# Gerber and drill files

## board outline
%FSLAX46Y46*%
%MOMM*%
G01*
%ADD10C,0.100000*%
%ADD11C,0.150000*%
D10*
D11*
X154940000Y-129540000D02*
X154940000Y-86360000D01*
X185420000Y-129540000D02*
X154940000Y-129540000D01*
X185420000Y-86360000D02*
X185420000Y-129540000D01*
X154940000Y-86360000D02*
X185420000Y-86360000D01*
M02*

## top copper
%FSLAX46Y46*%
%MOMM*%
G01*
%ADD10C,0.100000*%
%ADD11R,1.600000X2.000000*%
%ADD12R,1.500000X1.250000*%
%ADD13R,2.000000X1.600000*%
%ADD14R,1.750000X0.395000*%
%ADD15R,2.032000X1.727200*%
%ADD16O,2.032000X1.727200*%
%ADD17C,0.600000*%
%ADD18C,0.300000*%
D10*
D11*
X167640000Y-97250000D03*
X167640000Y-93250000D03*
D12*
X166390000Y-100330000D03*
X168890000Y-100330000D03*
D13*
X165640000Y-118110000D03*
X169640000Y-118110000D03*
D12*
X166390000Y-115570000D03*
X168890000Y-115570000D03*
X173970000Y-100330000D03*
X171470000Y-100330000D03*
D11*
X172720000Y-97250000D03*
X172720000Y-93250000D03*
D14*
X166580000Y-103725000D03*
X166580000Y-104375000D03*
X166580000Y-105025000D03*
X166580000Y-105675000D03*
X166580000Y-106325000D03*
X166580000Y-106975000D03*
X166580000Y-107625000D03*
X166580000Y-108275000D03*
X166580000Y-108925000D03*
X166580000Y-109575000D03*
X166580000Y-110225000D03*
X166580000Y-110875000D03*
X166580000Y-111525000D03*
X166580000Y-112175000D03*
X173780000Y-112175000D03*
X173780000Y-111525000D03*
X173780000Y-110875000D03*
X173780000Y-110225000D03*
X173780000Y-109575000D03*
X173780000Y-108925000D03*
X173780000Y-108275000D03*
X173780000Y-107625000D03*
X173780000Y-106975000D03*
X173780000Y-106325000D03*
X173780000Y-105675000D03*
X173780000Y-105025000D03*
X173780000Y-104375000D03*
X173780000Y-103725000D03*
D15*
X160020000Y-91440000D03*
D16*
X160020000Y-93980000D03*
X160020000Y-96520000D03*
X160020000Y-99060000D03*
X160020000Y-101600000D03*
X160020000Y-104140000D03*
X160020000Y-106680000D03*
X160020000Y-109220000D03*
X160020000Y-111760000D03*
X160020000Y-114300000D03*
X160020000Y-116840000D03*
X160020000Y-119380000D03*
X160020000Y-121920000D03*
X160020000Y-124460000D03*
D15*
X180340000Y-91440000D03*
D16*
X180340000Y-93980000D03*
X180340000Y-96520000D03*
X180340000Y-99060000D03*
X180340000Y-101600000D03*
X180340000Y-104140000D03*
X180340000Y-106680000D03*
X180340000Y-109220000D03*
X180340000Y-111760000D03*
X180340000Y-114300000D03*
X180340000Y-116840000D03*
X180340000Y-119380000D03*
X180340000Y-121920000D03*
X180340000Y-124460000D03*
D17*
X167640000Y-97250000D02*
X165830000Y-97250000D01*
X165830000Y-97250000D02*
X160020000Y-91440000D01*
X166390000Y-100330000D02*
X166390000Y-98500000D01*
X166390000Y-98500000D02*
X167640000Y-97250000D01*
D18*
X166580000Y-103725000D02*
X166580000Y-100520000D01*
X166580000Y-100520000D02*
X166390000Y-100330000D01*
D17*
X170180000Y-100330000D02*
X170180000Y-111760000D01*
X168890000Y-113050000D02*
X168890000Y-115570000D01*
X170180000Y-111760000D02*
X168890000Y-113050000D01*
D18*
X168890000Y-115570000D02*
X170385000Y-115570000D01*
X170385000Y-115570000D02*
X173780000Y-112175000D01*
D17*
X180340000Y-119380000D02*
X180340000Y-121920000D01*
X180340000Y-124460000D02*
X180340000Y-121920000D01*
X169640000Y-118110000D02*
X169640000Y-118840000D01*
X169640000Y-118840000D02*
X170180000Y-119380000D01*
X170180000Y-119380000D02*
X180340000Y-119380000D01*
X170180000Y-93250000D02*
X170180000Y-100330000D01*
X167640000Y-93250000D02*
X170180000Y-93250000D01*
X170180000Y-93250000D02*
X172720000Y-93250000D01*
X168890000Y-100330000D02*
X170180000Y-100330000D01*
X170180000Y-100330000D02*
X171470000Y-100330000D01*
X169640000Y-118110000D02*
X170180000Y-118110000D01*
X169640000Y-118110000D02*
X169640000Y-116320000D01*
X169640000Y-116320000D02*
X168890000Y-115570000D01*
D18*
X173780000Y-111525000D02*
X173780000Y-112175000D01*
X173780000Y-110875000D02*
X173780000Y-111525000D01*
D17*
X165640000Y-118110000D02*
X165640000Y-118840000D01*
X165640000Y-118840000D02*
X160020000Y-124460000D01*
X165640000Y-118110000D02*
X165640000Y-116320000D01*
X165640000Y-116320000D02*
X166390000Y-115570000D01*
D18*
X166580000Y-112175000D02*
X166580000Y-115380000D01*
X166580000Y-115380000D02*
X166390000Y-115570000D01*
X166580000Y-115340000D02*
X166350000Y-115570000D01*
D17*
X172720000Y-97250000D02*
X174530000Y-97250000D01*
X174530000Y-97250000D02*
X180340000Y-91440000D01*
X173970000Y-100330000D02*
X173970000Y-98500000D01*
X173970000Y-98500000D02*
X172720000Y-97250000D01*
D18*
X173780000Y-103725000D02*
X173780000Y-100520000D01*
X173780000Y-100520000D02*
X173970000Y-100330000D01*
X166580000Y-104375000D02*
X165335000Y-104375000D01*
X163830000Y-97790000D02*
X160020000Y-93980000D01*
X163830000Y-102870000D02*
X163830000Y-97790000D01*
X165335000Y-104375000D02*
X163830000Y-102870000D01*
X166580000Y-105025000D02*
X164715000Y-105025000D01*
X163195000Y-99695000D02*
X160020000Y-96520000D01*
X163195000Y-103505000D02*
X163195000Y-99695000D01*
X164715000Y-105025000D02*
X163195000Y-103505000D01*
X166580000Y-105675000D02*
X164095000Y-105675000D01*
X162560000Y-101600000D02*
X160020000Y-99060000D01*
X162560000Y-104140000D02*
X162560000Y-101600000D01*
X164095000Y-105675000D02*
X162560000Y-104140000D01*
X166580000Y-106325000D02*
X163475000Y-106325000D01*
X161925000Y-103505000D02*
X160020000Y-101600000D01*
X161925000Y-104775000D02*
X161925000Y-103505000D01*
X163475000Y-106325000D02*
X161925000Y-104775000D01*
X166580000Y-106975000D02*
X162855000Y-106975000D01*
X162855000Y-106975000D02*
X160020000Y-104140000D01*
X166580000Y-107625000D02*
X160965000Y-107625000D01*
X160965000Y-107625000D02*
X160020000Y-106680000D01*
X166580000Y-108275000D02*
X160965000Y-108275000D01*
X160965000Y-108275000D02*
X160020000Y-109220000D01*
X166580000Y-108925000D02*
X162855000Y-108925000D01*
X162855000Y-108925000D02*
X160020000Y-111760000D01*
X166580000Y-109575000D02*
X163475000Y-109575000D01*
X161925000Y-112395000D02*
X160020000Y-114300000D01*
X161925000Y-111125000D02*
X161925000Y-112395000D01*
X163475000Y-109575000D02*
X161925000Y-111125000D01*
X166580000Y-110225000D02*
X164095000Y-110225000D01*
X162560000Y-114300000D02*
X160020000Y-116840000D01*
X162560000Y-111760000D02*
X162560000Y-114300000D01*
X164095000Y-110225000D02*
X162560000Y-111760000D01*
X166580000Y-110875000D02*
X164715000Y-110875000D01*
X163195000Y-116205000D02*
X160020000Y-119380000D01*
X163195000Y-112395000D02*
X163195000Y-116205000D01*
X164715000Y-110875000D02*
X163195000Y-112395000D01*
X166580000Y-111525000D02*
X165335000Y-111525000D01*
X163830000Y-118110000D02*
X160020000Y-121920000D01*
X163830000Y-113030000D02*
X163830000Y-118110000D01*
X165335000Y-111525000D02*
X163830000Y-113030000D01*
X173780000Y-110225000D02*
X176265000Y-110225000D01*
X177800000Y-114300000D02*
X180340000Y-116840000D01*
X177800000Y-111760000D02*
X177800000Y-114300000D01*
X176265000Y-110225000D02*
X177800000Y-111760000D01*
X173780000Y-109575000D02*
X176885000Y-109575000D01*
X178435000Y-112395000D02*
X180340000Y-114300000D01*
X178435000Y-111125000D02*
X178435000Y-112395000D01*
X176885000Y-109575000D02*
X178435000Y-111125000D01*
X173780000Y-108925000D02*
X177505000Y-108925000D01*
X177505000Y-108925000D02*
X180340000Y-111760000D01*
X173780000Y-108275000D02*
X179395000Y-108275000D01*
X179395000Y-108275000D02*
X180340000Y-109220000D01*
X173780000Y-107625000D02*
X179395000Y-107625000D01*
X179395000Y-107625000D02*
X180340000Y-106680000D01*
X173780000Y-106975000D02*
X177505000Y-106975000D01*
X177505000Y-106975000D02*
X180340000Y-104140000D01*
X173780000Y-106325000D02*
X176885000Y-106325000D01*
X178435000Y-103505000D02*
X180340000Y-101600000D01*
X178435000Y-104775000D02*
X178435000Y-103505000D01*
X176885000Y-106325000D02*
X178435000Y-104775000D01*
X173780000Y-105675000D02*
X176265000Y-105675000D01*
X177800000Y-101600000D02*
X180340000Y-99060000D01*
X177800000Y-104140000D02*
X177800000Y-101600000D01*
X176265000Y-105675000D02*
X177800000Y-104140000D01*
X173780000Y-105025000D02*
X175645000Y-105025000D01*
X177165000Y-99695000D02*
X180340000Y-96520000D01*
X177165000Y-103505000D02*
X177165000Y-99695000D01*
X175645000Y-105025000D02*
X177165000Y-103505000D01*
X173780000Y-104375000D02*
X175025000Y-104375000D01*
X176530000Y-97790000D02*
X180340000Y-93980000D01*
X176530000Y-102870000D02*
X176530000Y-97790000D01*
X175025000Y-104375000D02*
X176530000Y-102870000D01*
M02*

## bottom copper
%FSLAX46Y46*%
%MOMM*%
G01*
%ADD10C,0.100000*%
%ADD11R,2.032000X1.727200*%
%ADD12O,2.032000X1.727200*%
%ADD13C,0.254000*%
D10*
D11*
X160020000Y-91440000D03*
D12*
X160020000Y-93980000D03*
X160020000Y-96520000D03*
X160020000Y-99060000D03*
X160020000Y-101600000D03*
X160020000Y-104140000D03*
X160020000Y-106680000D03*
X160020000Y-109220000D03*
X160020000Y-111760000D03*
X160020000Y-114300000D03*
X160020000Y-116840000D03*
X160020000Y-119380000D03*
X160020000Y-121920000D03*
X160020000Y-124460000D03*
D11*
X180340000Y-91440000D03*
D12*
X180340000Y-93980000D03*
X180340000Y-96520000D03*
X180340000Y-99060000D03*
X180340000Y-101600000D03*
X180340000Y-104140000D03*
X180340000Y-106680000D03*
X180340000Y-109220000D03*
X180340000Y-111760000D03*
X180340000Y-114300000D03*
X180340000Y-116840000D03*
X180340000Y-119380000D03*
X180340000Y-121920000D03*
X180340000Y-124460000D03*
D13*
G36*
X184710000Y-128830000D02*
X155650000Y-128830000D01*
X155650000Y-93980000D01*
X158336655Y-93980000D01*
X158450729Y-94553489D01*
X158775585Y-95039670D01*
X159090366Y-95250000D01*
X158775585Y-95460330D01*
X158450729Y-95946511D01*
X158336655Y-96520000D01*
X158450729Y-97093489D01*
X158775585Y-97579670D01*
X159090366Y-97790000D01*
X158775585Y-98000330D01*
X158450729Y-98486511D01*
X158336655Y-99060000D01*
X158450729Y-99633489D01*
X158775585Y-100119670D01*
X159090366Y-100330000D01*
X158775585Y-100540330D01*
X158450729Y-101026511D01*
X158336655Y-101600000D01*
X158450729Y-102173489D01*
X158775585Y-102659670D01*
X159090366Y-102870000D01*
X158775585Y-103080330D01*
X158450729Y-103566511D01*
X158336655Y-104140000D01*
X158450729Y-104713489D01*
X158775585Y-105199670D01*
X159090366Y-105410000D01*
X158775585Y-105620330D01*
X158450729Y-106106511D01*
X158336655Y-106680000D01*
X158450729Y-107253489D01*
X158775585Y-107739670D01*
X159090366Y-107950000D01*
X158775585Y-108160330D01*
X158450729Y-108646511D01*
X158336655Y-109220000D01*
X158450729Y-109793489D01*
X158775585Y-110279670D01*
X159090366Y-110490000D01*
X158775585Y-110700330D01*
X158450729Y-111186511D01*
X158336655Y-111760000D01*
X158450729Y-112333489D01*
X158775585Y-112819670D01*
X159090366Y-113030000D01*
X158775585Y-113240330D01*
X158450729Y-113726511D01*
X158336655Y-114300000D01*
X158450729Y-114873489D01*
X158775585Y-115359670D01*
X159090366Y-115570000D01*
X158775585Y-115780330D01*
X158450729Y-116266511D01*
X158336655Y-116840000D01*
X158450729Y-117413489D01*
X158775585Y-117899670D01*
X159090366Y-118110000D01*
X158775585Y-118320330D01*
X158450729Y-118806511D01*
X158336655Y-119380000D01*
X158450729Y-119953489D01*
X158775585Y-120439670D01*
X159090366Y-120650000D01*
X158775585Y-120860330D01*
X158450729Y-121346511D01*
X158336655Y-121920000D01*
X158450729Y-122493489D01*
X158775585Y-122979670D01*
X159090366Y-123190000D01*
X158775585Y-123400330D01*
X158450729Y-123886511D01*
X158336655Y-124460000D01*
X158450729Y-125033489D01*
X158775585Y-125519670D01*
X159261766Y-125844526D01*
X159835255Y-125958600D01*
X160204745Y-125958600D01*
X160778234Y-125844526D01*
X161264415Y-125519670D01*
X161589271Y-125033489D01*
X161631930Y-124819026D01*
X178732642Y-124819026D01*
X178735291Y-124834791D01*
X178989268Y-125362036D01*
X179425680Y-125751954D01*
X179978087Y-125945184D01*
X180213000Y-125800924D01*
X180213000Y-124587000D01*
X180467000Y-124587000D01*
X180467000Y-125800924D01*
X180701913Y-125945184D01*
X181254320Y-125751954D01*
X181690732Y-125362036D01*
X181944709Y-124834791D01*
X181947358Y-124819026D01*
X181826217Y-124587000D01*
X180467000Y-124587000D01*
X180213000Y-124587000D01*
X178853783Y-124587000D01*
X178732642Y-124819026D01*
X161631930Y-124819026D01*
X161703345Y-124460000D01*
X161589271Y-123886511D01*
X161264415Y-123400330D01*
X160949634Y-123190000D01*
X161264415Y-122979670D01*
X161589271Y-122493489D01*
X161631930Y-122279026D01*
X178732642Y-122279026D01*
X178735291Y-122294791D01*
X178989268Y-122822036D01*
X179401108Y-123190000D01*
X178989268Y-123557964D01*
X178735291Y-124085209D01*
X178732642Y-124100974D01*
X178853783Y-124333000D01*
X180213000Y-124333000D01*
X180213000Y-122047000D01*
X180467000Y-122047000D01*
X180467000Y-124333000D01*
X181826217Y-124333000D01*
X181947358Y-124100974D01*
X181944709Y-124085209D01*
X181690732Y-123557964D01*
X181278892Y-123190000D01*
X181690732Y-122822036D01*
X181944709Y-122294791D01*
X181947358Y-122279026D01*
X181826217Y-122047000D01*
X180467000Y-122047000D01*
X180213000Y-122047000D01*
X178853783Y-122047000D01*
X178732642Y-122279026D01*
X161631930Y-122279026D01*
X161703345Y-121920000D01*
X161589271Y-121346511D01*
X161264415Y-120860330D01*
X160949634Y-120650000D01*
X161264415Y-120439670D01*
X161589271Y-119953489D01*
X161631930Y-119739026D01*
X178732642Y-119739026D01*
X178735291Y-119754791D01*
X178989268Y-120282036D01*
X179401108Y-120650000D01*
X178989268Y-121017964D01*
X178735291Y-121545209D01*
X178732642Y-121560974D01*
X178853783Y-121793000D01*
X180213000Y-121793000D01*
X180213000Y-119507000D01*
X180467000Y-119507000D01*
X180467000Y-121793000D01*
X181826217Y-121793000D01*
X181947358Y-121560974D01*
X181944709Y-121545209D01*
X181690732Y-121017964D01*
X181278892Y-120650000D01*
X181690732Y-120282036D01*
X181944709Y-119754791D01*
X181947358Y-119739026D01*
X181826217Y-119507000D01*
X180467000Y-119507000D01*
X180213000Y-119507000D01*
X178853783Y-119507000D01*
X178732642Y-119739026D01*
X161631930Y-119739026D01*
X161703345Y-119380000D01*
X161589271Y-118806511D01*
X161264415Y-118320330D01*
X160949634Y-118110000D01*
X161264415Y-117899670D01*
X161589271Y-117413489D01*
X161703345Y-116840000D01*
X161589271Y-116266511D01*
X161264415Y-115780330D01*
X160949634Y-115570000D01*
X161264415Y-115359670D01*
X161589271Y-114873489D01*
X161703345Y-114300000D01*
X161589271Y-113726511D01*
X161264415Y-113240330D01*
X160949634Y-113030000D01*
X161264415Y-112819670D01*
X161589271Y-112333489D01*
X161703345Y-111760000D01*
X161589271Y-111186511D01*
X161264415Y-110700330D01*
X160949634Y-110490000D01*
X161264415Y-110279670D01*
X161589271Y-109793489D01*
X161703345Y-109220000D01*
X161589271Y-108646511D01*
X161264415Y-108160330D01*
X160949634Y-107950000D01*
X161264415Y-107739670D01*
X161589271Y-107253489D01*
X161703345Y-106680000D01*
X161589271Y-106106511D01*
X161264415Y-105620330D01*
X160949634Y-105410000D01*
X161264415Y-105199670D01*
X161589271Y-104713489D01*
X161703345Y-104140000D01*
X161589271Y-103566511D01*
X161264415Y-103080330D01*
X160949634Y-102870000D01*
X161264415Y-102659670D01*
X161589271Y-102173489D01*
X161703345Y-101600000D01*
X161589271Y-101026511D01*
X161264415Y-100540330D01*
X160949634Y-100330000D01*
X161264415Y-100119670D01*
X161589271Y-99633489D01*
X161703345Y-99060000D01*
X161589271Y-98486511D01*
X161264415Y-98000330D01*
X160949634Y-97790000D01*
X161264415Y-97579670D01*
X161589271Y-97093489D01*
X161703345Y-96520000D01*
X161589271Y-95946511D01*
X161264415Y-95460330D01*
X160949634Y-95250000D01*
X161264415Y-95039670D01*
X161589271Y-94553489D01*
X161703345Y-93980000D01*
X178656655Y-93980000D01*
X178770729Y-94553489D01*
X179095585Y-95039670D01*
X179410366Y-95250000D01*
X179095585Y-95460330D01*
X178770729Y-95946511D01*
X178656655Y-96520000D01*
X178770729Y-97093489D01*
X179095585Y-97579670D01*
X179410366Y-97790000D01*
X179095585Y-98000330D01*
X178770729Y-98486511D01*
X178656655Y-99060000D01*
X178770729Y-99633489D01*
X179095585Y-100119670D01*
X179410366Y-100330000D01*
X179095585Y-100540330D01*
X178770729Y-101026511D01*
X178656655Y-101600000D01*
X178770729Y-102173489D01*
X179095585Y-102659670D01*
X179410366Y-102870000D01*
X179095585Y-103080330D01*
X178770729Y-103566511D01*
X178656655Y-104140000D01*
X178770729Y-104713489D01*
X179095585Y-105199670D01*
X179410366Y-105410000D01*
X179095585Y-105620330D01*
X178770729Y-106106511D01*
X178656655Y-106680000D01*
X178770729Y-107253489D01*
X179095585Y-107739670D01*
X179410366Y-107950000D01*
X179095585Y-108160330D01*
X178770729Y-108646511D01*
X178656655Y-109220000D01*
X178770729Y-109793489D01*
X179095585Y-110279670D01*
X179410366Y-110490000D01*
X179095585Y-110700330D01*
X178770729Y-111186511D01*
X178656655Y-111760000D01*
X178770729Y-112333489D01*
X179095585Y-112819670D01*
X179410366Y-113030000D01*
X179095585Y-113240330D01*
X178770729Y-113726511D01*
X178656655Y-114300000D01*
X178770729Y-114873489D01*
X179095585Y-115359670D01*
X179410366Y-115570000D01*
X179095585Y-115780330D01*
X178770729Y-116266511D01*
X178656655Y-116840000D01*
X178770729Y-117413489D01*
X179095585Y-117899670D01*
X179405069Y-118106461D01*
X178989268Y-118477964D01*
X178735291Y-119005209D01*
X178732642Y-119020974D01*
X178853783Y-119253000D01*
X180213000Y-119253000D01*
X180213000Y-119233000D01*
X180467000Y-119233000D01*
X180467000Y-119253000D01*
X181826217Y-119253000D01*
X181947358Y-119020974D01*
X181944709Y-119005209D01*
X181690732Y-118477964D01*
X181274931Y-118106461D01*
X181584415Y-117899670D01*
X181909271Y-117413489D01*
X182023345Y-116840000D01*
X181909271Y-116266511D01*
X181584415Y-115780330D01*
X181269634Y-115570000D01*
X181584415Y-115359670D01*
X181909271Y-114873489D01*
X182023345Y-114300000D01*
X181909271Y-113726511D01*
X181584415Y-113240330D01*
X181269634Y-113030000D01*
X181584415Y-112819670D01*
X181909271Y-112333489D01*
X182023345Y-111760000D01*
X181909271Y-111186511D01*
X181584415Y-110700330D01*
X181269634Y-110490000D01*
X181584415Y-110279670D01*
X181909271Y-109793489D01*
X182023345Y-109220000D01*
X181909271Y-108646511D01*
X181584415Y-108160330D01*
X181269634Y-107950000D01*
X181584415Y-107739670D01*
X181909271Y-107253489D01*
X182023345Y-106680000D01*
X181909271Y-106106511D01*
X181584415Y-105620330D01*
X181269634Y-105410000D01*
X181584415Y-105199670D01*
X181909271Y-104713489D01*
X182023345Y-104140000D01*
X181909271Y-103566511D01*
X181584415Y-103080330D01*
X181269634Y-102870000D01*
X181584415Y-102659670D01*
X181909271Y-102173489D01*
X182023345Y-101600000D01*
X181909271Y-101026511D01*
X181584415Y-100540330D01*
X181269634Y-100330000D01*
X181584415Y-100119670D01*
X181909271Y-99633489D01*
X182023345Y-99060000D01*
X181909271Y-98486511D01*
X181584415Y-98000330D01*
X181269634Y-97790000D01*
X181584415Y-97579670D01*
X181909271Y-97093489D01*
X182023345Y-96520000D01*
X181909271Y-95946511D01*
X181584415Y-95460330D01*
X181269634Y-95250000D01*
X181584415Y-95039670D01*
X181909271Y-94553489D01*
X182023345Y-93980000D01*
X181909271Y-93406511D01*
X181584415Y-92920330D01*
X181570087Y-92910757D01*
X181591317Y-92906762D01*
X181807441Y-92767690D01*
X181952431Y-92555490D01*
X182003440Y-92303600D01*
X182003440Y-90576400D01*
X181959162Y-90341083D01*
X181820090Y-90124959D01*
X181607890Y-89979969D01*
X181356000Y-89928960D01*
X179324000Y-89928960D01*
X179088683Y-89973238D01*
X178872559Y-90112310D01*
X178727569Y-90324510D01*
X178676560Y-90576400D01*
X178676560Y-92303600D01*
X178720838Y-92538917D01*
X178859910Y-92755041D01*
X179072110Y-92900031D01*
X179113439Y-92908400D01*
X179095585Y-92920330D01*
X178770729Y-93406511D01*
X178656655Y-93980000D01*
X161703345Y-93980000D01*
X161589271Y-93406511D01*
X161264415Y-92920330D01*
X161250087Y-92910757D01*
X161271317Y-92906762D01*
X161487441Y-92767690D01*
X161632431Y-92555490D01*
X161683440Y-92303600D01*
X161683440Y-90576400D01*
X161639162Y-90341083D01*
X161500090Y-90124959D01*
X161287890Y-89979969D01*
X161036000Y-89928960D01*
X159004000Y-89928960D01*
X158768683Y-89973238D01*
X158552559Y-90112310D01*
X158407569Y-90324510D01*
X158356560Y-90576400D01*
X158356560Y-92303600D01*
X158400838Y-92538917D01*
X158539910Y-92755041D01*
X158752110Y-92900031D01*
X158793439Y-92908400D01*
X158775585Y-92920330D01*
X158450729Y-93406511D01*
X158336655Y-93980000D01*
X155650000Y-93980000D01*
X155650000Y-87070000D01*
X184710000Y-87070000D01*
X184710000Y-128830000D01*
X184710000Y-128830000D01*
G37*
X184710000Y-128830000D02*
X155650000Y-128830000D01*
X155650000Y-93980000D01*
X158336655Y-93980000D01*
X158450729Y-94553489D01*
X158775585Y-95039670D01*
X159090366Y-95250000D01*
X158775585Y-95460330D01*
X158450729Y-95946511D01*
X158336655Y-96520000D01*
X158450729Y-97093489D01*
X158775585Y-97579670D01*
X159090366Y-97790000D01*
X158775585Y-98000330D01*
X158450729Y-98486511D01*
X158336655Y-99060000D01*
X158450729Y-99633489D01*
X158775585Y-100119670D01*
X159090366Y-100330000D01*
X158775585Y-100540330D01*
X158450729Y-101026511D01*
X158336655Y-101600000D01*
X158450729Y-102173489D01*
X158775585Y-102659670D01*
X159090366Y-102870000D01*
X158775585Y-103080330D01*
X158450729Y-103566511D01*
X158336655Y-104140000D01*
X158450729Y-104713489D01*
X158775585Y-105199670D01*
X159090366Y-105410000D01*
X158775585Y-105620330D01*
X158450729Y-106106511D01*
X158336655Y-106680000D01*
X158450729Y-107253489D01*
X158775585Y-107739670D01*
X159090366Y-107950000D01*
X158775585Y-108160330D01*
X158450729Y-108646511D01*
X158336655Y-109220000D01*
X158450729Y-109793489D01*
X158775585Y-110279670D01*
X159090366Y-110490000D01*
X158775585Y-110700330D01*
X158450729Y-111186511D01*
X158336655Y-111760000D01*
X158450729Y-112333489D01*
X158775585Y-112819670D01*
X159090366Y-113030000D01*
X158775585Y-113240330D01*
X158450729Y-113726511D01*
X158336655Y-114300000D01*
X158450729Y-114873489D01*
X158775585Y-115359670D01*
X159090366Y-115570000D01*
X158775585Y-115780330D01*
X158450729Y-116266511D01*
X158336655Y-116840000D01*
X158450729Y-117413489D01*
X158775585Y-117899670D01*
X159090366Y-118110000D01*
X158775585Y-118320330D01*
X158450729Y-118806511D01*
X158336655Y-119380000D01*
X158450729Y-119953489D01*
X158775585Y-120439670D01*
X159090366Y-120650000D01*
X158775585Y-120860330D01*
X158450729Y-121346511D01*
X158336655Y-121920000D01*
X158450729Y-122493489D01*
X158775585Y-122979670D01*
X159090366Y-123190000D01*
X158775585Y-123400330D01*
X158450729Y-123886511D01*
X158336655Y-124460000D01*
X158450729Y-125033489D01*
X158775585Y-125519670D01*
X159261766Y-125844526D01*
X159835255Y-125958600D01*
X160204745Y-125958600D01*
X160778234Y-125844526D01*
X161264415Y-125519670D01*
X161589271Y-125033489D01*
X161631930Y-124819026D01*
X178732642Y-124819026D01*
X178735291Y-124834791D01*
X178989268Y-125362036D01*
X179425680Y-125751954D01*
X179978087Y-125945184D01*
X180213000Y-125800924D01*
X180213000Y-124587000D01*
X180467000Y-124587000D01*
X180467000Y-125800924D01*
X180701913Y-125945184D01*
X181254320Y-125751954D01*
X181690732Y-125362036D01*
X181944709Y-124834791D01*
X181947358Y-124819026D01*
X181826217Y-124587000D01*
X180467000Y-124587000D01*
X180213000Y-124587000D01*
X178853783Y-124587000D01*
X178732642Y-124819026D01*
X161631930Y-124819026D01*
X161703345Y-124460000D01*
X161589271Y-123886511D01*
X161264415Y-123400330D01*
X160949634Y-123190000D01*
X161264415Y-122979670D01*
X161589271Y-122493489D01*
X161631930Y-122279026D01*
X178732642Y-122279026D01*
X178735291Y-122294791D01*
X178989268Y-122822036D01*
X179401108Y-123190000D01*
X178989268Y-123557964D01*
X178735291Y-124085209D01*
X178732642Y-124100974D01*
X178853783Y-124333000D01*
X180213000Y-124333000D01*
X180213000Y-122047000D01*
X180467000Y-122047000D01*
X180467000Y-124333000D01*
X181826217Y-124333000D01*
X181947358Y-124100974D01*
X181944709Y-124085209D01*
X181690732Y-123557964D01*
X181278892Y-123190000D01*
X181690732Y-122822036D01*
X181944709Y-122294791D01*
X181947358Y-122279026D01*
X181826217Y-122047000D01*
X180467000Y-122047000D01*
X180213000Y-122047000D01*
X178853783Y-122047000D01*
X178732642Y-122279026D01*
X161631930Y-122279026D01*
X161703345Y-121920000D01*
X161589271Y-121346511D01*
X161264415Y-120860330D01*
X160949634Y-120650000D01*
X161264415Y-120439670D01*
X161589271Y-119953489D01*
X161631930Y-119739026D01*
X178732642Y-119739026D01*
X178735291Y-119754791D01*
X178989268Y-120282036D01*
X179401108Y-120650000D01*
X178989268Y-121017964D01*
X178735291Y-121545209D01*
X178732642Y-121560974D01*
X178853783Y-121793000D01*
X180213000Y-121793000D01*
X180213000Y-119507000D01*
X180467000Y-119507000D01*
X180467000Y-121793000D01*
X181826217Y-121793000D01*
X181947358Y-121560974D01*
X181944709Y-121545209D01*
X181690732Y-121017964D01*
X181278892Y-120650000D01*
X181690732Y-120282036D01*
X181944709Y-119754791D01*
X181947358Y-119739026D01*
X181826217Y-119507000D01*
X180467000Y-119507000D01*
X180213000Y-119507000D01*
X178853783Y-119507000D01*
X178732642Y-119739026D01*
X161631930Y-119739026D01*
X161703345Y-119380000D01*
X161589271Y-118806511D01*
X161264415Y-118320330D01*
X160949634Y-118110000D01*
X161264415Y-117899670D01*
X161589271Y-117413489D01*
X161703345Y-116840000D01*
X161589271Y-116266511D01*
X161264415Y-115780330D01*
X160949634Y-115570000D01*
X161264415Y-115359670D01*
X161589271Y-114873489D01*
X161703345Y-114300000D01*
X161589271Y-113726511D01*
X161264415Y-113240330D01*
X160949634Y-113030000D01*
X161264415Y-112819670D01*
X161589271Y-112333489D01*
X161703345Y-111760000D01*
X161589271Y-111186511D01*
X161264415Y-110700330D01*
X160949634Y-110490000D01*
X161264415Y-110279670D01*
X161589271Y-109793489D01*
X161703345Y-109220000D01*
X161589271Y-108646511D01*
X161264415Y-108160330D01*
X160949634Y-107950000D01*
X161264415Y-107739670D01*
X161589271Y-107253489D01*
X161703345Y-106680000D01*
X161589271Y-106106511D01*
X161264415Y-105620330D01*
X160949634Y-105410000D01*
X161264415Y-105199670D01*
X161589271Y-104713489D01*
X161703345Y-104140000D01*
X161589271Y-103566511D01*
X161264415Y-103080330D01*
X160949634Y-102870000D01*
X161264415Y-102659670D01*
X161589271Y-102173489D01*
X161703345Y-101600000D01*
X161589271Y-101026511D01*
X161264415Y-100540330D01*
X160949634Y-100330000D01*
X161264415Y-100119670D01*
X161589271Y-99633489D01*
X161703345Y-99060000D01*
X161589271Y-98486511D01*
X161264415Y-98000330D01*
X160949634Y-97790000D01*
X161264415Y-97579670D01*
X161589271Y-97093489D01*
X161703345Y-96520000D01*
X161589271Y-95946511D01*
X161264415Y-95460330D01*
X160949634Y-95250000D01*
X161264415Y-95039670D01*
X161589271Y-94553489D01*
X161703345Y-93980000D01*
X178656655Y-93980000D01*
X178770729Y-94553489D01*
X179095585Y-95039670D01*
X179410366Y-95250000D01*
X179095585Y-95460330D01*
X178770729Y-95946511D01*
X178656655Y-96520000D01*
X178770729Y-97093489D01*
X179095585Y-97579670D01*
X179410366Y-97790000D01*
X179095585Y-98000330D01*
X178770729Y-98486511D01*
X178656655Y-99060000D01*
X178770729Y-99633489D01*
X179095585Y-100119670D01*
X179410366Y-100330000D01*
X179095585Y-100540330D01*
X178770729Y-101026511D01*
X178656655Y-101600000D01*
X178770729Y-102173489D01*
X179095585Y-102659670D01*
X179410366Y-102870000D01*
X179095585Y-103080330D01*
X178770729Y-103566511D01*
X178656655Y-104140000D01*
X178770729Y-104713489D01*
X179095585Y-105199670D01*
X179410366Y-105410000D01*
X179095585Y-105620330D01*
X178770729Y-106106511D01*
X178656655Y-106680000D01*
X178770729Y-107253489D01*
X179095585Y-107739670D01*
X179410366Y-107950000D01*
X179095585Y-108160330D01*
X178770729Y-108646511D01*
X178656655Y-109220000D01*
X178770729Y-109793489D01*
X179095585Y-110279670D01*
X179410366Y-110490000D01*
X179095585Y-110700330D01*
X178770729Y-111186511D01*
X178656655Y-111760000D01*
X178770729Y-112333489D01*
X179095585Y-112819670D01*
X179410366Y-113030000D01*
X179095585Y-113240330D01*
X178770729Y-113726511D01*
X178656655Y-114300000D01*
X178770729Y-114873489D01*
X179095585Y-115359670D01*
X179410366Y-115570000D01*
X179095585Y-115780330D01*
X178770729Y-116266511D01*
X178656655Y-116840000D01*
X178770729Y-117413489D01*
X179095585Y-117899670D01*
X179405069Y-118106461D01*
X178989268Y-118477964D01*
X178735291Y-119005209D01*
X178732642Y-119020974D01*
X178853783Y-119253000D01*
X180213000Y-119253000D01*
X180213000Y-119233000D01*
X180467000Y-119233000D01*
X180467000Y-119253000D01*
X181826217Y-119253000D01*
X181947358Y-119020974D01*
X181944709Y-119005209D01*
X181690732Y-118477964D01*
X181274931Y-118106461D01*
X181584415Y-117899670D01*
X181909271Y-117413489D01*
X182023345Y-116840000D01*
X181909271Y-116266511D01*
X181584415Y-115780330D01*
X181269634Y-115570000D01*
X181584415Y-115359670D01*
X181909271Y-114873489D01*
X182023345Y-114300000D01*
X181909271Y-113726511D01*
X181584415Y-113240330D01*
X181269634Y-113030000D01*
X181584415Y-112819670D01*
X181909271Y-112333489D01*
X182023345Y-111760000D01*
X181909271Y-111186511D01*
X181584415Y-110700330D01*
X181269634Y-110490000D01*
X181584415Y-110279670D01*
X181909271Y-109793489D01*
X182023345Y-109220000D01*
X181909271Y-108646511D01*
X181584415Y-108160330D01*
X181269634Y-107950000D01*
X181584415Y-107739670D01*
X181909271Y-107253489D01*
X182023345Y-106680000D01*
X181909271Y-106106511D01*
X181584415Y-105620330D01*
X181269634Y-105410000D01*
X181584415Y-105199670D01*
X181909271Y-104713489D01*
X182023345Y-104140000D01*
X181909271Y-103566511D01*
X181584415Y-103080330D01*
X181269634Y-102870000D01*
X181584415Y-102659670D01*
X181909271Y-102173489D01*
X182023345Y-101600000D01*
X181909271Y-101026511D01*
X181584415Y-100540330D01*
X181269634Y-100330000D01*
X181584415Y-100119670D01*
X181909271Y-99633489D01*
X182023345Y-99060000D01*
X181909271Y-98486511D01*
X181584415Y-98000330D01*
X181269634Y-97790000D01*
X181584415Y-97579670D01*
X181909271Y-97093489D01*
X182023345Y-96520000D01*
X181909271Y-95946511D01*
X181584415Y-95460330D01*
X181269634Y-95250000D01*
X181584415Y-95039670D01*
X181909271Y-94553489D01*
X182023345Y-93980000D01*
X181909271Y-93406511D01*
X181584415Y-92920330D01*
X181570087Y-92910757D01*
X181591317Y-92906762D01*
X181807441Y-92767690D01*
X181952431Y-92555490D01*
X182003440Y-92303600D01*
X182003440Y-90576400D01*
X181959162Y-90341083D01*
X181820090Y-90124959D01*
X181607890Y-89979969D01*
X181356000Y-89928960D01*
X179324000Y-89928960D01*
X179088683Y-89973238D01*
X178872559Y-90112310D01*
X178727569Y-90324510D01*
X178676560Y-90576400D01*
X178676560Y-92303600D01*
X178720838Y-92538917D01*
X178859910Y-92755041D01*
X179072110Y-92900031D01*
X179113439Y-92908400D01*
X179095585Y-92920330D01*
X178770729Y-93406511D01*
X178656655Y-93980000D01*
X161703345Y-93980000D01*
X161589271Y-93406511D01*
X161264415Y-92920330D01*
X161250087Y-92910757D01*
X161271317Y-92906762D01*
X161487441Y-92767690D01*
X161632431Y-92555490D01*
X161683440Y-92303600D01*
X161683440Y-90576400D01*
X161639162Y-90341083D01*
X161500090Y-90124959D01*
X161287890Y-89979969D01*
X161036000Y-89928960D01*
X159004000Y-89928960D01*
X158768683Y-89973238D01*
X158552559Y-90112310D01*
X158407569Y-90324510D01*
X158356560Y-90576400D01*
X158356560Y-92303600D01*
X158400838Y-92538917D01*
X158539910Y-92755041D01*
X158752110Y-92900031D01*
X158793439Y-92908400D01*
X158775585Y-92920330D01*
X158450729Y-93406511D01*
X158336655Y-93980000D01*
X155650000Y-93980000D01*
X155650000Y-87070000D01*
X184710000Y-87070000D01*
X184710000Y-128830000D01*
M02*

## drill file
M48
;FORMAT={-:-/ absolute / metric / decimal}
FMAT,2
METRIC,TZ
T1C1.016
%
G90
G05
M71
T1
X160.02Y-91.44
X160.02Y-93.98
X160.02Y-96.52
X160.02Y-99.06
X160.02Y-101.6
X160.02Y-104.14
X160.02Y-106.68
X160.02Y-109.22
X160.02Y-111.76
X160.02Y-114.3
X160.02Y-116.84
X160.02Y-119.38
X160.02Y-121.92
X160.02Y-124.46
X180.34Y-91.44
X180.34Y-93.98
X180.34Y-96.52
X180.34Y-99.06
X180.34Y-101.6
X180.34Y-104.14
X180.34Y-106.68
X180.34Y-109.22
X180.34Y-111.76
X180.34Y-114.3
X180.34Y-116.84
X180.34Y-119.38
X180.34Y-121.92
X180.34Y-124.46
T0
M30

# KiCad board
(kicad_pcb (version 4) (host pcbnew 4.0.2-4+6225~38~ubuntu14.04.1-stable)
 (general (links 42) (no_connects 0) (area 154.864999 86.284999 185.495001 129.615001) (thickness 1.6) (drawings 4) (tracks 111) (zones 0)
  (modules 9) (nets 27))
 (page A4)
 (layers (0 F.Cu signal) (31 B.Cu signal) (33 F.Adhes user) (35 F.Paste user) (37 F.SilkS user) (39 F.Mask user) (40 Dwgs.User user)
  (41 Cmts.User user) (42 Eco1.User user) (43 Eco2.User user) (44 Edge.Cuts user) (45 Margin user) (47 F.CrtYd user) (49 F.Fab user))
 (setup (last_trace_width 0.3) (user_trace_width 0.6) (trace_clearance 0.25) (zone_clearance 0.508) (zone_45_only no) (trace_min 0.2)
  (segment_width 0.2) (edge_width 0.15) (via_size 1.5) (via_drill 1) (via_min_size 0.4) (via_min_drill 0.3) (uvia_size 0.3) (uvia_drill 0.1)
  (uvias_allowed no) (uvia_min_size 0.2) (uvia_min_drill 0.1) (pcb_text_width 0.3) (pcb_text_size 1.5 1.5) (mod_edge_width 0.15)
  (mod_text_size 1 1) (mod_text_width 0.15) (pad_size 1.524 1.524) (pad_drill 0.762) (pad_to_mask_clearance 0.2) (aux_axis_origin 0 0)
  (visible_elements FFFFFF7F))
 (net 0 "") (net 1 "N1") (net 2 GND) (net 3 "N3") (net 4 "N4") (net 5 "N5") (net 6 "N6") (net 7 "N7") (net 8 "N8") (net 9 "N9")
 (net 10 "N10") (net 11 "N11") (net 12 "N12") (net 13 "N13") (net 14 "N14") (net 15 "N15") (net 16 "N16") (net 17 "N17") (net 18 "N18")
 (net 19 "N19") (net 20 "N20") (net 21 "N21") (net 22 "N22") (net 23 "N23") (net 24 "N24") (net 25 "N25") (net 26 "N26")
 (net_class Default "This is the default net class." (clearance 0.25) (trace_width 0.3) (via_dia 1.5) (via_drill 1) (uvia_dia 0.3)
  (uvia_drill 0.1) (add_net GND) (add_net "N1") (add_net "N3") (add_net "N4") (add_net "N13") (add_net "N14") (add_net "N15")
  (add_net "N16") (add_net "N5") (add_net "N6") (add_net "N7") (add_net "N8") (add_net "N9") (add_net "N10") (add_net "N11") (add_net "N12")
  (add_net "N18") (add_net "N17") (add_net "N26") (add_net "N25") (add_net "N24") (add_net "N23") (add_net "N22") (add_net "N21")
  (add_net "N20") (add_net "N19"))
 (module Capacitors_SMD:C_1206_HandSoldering (layer F.Cu) (at 167.64 95.25 90)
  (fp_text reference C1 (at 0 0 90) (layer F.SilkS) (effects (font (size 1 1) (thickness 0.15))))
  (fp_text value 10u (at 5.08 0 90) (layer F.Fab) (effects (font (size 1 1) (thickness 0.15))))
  (pad 1 smd rect (at -2 0 90) (size 2 1.6) (layers F.Cu F.Paste F.Mask) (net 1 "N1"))
  (pad 2 smd rect (at 2 0 90) (size 2 1.6) (layers F.Cu F.Paste F.Mask) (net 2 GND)))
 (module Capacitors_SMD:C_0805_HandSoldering (layer F.Cu) (at 167.64 100.33)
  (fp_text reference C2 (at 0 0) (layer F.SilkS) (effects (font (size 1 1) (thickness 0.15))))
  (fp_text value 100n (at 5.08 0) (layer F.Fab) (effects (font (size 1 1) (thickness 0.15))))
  (pad 1 smd rect (at -1.25 0) (size 1.5 1.25) (layers F.Cu F.Paste F.Mask) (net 1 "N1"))
  (pad 2 smd rect (at 1.25 0) (size 1.5 1.25) (layers F.Cu F.Paste F.Mask) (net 2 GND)))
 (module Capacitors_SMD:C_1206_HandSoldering (layer F.Cu) (at 167.64 118.11)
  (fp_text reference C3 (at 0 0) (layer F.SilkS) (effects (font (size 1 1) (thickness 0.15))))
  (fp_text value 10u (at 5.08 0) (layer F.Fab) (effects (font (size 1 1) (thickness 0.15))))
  (pad 1 smd rect (at -2 0) (size 2 1.6) (layers F.Cu F.Paste F.Mask) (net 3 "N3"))
  (pad 2 smd rect (at 2 0) (size 2 1.6) (layers F.Cu F.Paste F.Mask) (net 2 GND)))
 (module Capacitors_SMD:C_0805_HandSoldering (layer F.Cu) (at 167.64 115.57)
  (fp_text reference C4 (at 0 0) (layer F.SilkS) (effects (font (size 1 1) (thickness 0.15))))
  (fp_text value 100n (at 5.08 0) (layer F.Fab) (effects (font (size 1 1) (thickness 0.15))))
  (pad 1 smd rect (at -1.25 0) (size 1.5 1.25) (layers F.Cu F.Paste F.Mask) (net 3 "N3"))
  (pad 2 smd rect (at 1.25 0) (size 1.5 1.25) (layers F.Cu F.Paste F.Mask) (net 2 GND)))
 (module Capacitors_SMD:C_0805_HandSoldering (layer F.Cu) (at 172.72 100.33 180)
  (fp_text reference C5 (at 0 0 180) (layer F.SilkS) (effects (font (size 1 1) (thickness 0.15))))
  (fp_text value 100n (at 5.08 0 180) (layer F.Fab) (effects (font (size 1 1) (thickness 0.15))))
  (pad 1 smd rect (at -1.25 0 180) (size 1.5 1.25) (layers F.Cu F.Paste F.Mask) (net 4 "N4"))
  (pad 2 smd rect (at 1.25 0 180) (size 1.5 1.25) (layers F.Cu F.Paste F.Mask) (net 2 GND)))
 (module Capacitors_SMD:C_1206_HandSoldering (layer F.Cu) (at 172.72 95.25 90)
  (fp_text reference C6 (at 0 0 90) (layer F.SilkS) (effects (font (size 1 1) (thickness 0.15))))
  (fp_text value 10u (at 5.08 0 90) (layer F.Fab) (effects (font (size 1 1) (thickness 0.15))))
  (pad 1 smd rect (at -2 0 90) (size 2 1.6) (layers F.Cu F.Paste F.Mask) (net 4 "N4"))
  (pad 2 smd rect (at 2 0 90) (size 2 1.6) (layers F.Cu F.Paste F.Mask) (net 2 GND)))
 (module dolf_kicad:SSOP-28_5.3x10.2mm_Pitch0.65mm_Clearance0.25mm (layer F.Cu) (at 170.18 107.95)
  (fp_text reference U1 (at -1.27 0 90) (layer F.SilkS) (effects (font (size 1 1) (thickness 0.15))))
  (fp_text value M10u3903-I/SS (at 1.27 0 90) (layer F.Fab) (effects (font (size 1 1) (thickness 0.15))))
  (pad 1 smd rect (at -3.6 -4.225) (size 1.75 0.395) (layers F.Cu F.Paste F.Mask) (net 1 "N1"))
  (pad 2 smd rect (at -3.6 -3.575) (size 1.75 0.395) (layers F.Cu F.Paste F.Mask) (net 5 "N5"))
  (pad 3 smd rect (at -3.6 -2.925) (size 1.75 0.395) (layers F.Cu F.Paste F.Mask) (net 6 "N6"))
  (pad 4 smd rect (at -3.6 -2.275) (size 1.75 0.395) (layers F.Cu F.Paste F.Mask) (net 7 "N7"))
  (pad 5 smd rect (at -3.6 -1.625) (size 1.75 0.395) (layers F.Cu F.Paste F.Mask) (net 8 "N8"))
  (pad 6 smd rect (at -3.6 -0.975) (size 1.75 0.395) (layers F.Cu F.Paste F.Mask) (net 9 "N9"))
  (pad 7 smd rect (at -3.6 -0.325) (size 1.75 0.395) (layers F.Cu F.Paste F.Mask) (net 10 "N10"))
  (pad 8 smd rect (at -3.6 0.325) (size 1.75 0.395) (layers F.Cu F.Paste F.Mask) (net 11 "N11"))
  (pad 9 smd rect (at -3.6 0.975) (size 1.75 0.395) (layers F.Cu F.Paste F.Mask) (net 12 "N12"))
  (pad 10 smd rect (at -3.6 1.625) (size 1.75 0.395) (layers F.Cu F.Paste F.Mask) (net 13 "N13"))
  (pad 11 smd rect (at -3.6 2.275) (size 1.75 0.395) (layers F.Cu F.Paste F.Mask) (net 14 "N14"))
  (pad 12 smd rect (at -3.6 2.925) (size 1.75 0.395) (layers F.Cu F.Paste F.Mask) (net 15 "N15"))
  (pad 13 smd rect (at -3.6 3.575) (size 1.75 0.395) (layers F.Cu F.Paste F.Mask) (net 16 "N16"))
  (pad 14 smd rect (at -3.6 4.225) (size 1.75 0.395) (layers F.Cu F.Paste F.Mask) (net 3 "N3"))
  (pad 15 smd rect (at 3.6 4.225) (size 1.75 0.395) (layers F.Cu F.Paste F.Mask) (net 2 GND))
  (pad 16 smd rect (at 3.6 3.575) (size 1.75 0.395) (layers F.Cu F.Paste F.Mask) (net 2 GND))
  (pad 17 smd rect (at 3.6 2.925) (size 1.75 0.395) (layers F.Cu F.Paste F.Mask) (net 2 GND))
  (pad 18 smd rect (at 3.6 2.275) (size 1.75 0.395) (layers F.Cu F.Paste F.Mask) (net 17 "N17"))
  (pad 19 smd rect (at 3.6 1.625) (size 1.75 0.395) (layers F.Cu F.Paste F.Mask) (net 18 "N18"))
  (pad 20 smd rect (at 3.6 0.975) (size 1.75 0.395) (layers F.Cu F.Paste F.Mask) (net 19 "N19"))
  (pad 21 smd rect (at 3.6 0.325) (size 1.75 0.395) (layers F.Cu F.Paste F.Mask) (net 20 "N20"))
  (pad 22 smd rect (at 3.6 -0.325) (size 1.75 0.395) (layers F.Cu F.Paste F.Mask) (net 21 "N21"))
  (pad 23 smd rect (at 3.6 -0.975) (size 1.75 0.395) (layers F.Cu F.Paste F.Mask) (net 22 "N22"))
  (pad 24 smd rect (at 3.6 -1.625) (size 1.75 0.395) (layers F.Cu F.Paste F.Mask) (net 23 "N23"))
  (pad 25 smd rect (at 3.6 -2.275) (size 1.75 0.395) (layers F.Cu F.Paste F.Mask) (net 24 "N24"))
  (pad 26 smd rect (at 3.6 -2.925) (size 1.75 0.395) (layers F.Cu F.Paste F.Mask) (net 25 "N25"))
  (pad 27 smd rect (at 3.6 -3.575) (size 1.75 0.395) (layers F.Cu F.Paste F.Mask) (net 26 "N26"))
  (pad 28 smd rect (at 3.6 -4.225) (size 1.75 0.395) (layers F.Cu F.Paste F.Mask) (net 4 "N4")))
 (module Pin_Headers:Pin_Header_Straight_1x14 (layer F.Cu) (at 160.02 91.44)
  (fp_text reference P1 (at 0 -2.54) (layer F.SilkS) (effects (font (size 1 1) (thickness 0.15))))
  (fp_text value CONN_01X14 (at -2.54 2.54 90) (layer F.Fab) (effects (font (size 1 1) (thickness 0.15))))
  (pad 1 thru_hole rect (at 0 0) (size 2.032 1.7272) (drill 1.016) (layers *.Cu *.Mask F.SilkS) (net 1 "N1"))
  (pad 2 thru_hole oval (at 0 2.54) (size 2.032 1.7272) (drill 1.016) (layers *.Cu *.Mask F.SilkS) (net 5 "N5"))
  (pad 3 thru_hole oval (at 0 5.08) (size 2.032 1.7272) (drill 1.016) (layers *.Cu *.Mask F.SilkS) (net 6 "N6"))
  (pad 4 thru_hole oval (at 0 7.62) (size 2.032 1.7272) (drill 1.016) (layers *.Cu *.Mask F.SilkS) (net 7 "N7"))
  (pad 5 thru_hole oval (at 0 10.16) (size 2.032 1.7272) (drill 1.016) (layers *.Cu *.Mask F.SilkS) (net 8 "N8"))
  (pad 6 thru_hole oval (at 0 12.7) (size 2.032 1.7272) (drill 1.016) (layers *.Cu *.Mask F.SilkS) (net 9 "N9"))
  (pad 7 thru_hole oval (at 0 15.24) (size 2.032 1.7272) (drill 1.016) (layers *.Cu *.Mask F.SilkS) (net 10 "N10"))
  (pad 8 thru_hole oval (at 0 17.78) (size 2.032 1.7272) (drill 1.016) (layers *.Cu *.Mask F.SilkS) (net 11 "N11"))
  (pad 9 thru_hole oval (at 0 20.32) (size 2.032 1.7272) (drill 1.016) (layers *.Cu *.Mask F.SilkS) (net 12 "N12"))
  (pad 10 thru_hole oval (at 0 22.86) (size 2.032 1.7272) (drill 1.016) (layers *.Cu *.Mask F.SilkS) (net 13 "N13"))
  (pad 11 thru_hole oval (at 0 25.4) (size 2.032 1.7272) (drill 1.016) (layers *.Cu *.Mask F.SilkS) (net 14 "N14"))
  (pad 12 thru_hole oval (at 0 27.94) (size 2.032 1.7272) (drill 1.016) (layers *.Cu *.Mask F.SilkS) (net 15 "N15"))
  (pad 13 thru_hole oval (at 0 30.48) (size 2.032 1.7272) (drill 1.016) (layers *.Cu *.Mask F.SilkS) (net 16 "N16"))
  (pad 14 thru_hole oval (at 0 33.02) (size 2.032 1.7272) (drill 1.016) (layers *.Cu *.Mask F.SilkS) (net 3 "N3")))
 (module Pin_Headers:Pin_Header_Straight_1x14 (layer F.Cu) (at 180.34 91.44)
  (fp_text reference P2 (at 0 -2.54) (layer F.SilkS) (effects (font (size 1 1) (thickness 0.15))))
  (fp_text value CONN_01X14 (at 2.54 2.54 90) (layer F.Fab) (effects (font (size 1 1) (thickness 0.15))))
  (pad 1 thru_hole rect (at 0 0) (size 2.032 1.7272) (drill 1.016) (layers *.Cu *.Mask F.SilkS) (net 4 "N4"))
  (pad 2 thru_hole oval (at 0 2.54) (size 2.032 1.7272) (drill 1.016) (layers *.Cu *.Mask F.SilkS) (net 26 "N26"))
  (pad 3 thru_hole oval (at 0 5.08) (size 2.032 1.7272) (drill 1.016) (layers *.Cu *.Mask F.SilkS) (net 25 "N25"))
  (pad 4 thru_hole oval (at 0 7.62) (size 2.032 1.7272) (drill 1.016) (layers *.Cu *.Mask F.SilkS) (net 24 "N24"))
  (pad 5 thru_hole oval (at 0 10.16) (size 2.032 1.7272) (drill 1.016) (layers *.Cu *.Mask F.SilkS) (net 23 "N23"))
  (pad 6 thru_hole oval (at 0 12.7) (size 2.032 1.7272) (drill 1.016) (layers *.Cu *.Mask F.SilkS) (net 22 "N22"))
  (pad 7 thru_hole oval (at 0 15.24) (size 2.032 1.7272) (drill 1.016) (layers *.Cu *.Mask F.SilkS) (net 21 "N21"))
  (pad 8 thru_hole oval (at 0 17.78) (size 2.032 1.7272) (drill 1.016) (layers *.Cu *.Mask F.SilkS) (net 20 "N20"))
  (pad 9 thru_hole oval (at 0 20.32) (size 2.032 1.7272) (drill 1.016) (layers *.Cu *.Mask F.SilkS) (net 19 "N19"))
  (pad 10 thru_hole oval (at 0 22.86) (size 2.032 1.7272) (drill 1.016) (layers *.Cu *.Mask F.SilkS) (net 18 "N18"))
  (pad 11 thru_hole oval (at 0 25.4) (size 2.032 1.7272) (drill 1.016) (layers *.Cu *.Mask F.SilkS) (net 17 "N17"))
  (pad 12 thru_hole oval (at 0 27.94) (size 2.032 1.7272) (drill 1.016) (layers *.Cu *.Mask F.SilkS) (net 2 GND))
  (pad 13 thru_hole oval (at 0 30.48) (size 2.032 1.7272) (drill 1.016) (layers *.Cu *.Mask F.SilkS) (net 2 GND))
  (pad 14 thru_hole oval (at 0 33.02) (size 2.032 1.7272) (drill 1.016) (layers *.Cu *.Mask F.SilkS) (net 2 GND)))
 (gr_line (start 154.94 129.54) (end 154.94 86.36) (angle 90) (layer Edge.Cuts) (width 0.15))
 (gr_line (start 185.42 129.54) (end 154.94 129.54) (angle 90) (layer Edge.Cuts) (width 0.15))
 (gr_line (start 185.42 86.36) (end 185.42 129.54) (angle 90) (layer Edge.Cuts) (width 0.15))
 (gr_line (start 154.94 86.36) (end 185.42 86.36) (angle 90) (layer Edge.Cuts) (width 0.15))
 (segment (start 167.64 97.25) (end 165.83 97.25) (width 0.6) (layer F.Cu) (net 1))
 (segment (start 165.83 97.25) (end 160.02 91.44) (width 0.6) (layer F.Cu) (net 1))
 (segment (start 166.39 100.33) (end 166.39 98.5) (width 0.6) (layer F.Cu) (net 1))
 (segment (start 166.39 98.5) (end 167.64 97.25) (width 0.6) (layer F.Cu) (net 1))
 (segment (start 166.58 103.725) (end 166.58 100.52) (width 0.3) (layer F.Cu) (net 1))
 (segment (start 166.58 100.52) (end 166.39 100.33) (width 0.3) (layer F.Cu) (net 1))
 (segment (start 170.18 100.33) (end 170.18 111.76) (width 0.6) (layer F.Cu) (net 2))
 (segment (start 168.89 113.05) (end 168.89 115.57) (width 0.6) (layer F.Cu) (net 2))
 (segment (start 170.18 111.76) (end 168.89 113.05) (width 0.6) (layer F.Cu) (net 2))
 (segment (start 168.89 115.57) (end 170.385 115.57) (width 0.3) (layer F.Cu) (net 2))
 (segment (start 170.385 115.57) (end 173.78 112.175) (width 0.3) (layer F.Cu) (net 2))
 (segment (start 180.34 119.38) (end 180.34 121.92) (width 0.6) (layer F.Cu) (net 2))
 (segment (start 180.34 124.46) (end 180.34 121.92) (width 0.6) (layer F.Cu) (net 2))
 (segment (start 169.64 118.11) (end 169.64 118.84) (width 0.6) (layer F.Cu) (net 2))
 (segment (start 169.64 118.84) (end 170.18 119.38) (width 0.6) (layer F.Cu) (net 2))
 (segment (start 170.18 119.38) (end 180.34 119.38) (width 0.6) (layer F.Cu) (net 2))
 (segment (start 170.18 93.25) (end 170.18 100.33) (width 0.6) (layer F.Cu) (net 2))
 (segment (start 167.64 93.25) (end 170.18 93.25) (width 0.6) (layer F.Cu) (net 2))
 (segment (start 170.18 93.25) (end 172.72 93.25) (width 0.6) (layer F.Cu) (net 2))
 (segment (start 168.89 100.33) (end 170.18 100.33) (width 0.6) (layer F.Cu) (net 2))
 (segment (start 170.18 100.33) (end 171.47 100.33) (width 0.6) (layer F.Cu) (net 2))
 (segment (start 169.64 118.11) (end 170.18 118.11) (width 0.6) (layer F.Cu) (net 2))
 (segment (start 169.64 118.11) (end 169.64 116.32) (width 0.6) (layer F.Cu) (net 2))
 (segment (start 169.64 116.32) (end 168.89 115.57) (width 0.6) (layer F.Cu) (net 2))
 (segment (start 173.78 111.525) (end 173.78 112.175) (width 0.3) (layer F.Cu) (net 2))
 (segment (start 173.78 110.875) (end 173.78 111.525) (width 0.3) (layer F.Cu) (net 2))
 (segment (start 165.64 118.11) (end 165.64 118.84) (width 0.6) (layer F.Cu) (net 3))
 (segment (start 165.64 118.84) (end 160.02 124.46) (width 0.6) (layer F.Cu) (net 3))
 (segment (start 165.64 118.11) (end 165.64 116.32) (width 0.6) (layer F.Cu) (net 3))
 (segment (start 165.64 116.32) (end 166.39 115.57) (width 0.6) (layer F.Cu) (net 3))
 (segment (start 166.58 112.175) (end 166.58 115.38) (width 0.3) (layer F.Cu) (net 3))
 (segment (start 166.58 115.38) (end 166.39 115.57) (width 0.3) (layer F.Cu) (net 3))
 (segment (start 166.58 115.34) (end 166.35 115.57) (width 0.3) (layer F.Cu) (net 3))
 (segment (start 172.72 97.25) (end 174.53 97.25) (width 0.6) (layer F.Cu) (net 4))
 (segment (start 174.53 97.25) (end 180.34 91.44) (width 0.6) (layer F.Cu) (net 4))
 (segment (start 173.97 100.33) (end 173.97 98.5) (width 0.6) (layer F.Cu) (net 4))
 (segment (start 173.97 98.5) (end 172.72 97.25) (width 0.6) (layer F.Cu) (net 4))
 (segment (start 173.78 103.725) (end 173.78 100.52) (width 0.3) (layer F.Cu) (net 4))
 (segment (start 173.78 100.52) (end 173.97 100.33) (width 0.3) (layer F.Cu) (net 4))
 (segment (start 166.58 104.375) (end 165.335 104.375) (width 0.3) (layer F.Cu) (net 5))
 (segment (start 163.83 97.79) (end 160.02 93.98) (width 0.3) (layer F.Cu) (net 5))
 (segment (start 163.83 102.87) (end 163.83 97.79) (width 0.3) (layer F.Cu) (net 5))
 (segment (start 165.335 104.375) (end 163.83 102.87) (width 0.3) (layer F.Cu) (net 5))
 (segment (start 166.58 105.025) (end 164.715 105.025) (width 0.3) (layer F.Cu) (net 6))
 (segment (start 163.195 99.695) (end 160.02 96.52) (width 0.3) (layer F.Cu) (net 6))
 (segment (start 163.195 103.505) (end 163.195 99.695) (width 0.3) (layer F.Cu) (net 6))
 (segment (start 164.715 105.025) (end 163.195 103.505) (width 0.3) (layer F.Cu) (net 6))
 (segment (start 166.58 105.675) (end 164.095 105.675) (width 0.3) (layer F.Cu) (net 7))
 (segment (start 162.56 101.6) (end 160.02 99.06) (width 0.3) (layer F.Cu) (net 7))
 (segment (start 162.56 104.14) (end 162.56 101.6) (width 0.3) (layer F.Cu) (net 7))
 (segment (start 164.095 105.675) (end 162.56 104.14) (width 0.3) (layer F.Cu) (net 7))
 (segment (start 166.58 106.325) (end 163.475 106.325) (width 0.3) (layer F.Cu) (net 8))
 (segment (start 161.925 103.505) (end 160.02 101.6) (width 0.3) (layer F.Cu) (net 8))
 (segment (start 161.925 104.775) (end 161.925 103.505) (width 0.3) (layer F.Cu) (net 8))
 (segment (start 163.475 106.325) (end 161.925 104.775) (width 0.3) (layer F.Cu) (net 8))
 (segment (start 166.58 106.975) (end 162.855 106.975) (width 0.3) (layer F.Cu) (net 9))
 (segment (start 162.855 106.975) (end 160.02 104.14) (width 0.3) (layer F.Cu) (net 9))
 (segment (start 166.58 107.625) (end 160.965 107.625) (width 0.3) (layer F.Cu) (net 10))
 (segment (start 160.965 107.625) (end 160.02 106.68) (width 0.3) (layer F.Cu) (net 10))
 (segment (start 166.58 108.275) (end 160.965 108.275) (width 0.3) (layer F.Cu) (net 11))
 (segment (start 160.965 108.275) (end 160.02 109.22) (width 0.3) (layer F.Cu) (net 11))
 (segment (start 166.58 108.925) (end 162.855 108.925) (width 0.3) (layer F.Cu) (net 12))
 (segment (start 162.855 108.925) (end 160.02 111.76) (width 0.3) (layer F.Cu) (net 12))
 (segment (start 166.58 109.575) (end 163.475 109.575) (width 0.3) (layer F.Cu) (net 13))
 (segment (start 161.925 112.395) (end 160.02 114.3) (width 0.3) (layer F.Cu) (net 13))
 (segment (start 161.925 111.125) (end 161.925 112.395) (width 0.3) (layer F.Cu) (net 13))
 (segment (start 163.475 109.575) (end 161.925 111.125) (width 0.3) (layer F.Cu) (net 13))
 (segment (start 166.58 110.225) (end 164.095 110.225) (width 0.3) (layer F.Cu) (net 14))
 (segment (start 162.56 114.3) (end 160.02 116.84) (width 0.3) (layer F.Cu) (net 14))
 (segment (start 162.56 111.76) (end 162.56 114.3) (width 0.3) (layer F.Cu) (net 14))
 (segment (start 164.095 110.225) (end 162.56 111.76) (width 0.3) (layer F.Cu) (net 14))
 (segment (start 166.58 110.875) (end 164.715 110.875) (width 0.3) (layer F.Cu) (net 15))
 (segment (start 163.195 116.205) (end 160.02 119.38) (width 0.3) (layer F.Cu) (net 15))
 (segment (start 163.195 112.395) (end 163.195 116.205) (width 0.3) (layer F.Cu) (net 15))
 (segment (start 164.715 110.875) (end 163.195 112.395) (width 0.3) (layer F.Cu) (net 15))
 (segment (start 166.58 111.525) (end 165.335 111.525) (width 0.3) (layer F.Cu) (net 16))
 (segment (start 163.83 118.11) (end 160.02 121.92) (width 0.3) (layer F.Cu) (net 16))
 (segment (start 163.83 113.03) (end 163.83 118.11) (width 0.3) (layer F.Cu) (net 16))
 (segment (start 165.335 111.525) (end 163.83 113.03) (width 0.3) (layer F.Cu) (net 16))
 (segment (start 173.78 110.225) (end 176.265 110.225) (width 0.3) (layer F.Cu) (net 17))
 (segment (start 177.8 114.3) (end 180.34 116.84) (width 0.3) (layer F.Cu) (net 17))
 (segment (start 177.8 111.76) (end 177.8 114.3) (width 0.3) (layer F.Cu) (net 17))
 (segment (start 176.265 110.225) (end 177.8 111.76) (width 0.3) (layer F.Cu) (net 17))
 (segment (start 173.78 109.575) (end 176.885 109.575) (width 0.3) (layer F.Cu) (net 18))
 (segment (start 178.435 112.395) (end 180.34 114.3) (width 0.3) (layer F.Cu) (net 18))
 (segment (start 178.435 111.125) (end 178.435 112.395) (width 0.3) (layer F.Cu) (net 18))
 (segment (start 176.885 109.575) (end 178.435 111.125) (width 0.3) (layer F.Cu) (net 18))
 (segment (start 173.78 108.925) (end 177.505 108.925) (width 0.3) (layer F.Cu) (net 19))
 (segment (start 177.505 108.925) (end 180.34 111.76) (width 0.3) (layer F.Cu) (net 19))
 (segment (start 173.78 108.275) (end 179.395 108.275) (width 0.3) (layer F.Cu) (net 20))
 (segment (start 179.395 108.275) (end 180.34 109.22) (width 0.3) (layer F.Cu) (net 20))
 (segment (start 173.78 107.625) (end 179.395 107.625) (width 0.3) (layer F.Cu) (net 21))
 (segment (start 179.395 107.625) (end 180.34 106.68) (width 0.3) (layer F.Cu) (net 21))
 (segment (start 173.78 106.975) (end 177.505 106.975) (width 0.3) (layer F.Cu) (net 22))
 (segment (start 177.505 106.975) (end 180.34 104.14) (width 0.3) (layer F.Cu) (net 22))
 (segment (start 173.78 106.325) (end 176.885 106.325) (width 0.3) (layer F.Cu) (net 23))
 (segment (start 178.435 103.505) (end 180.34 101.6) (width 0.3) (layer F.Cu) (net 23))
 (segment (start 178.435 104.775) (end 178.435 103.505) (width 0.3) (layer F.Cu) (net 23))
 (segment (start 176.885 106.325) (end 178.435 104.775) (width 0.3) (layer F.Cu) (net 23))
 (segment (start 173.78 105.675) (end 176.265 105.675) (width 0.3) (layer F.Cu) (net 24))
 (segment (start 177.8 101.6) (end 180.34 99.06) (width 0.3) (layer F.Cu) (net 24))
 (segment (start 177.8 104.14) (end 177.8 101.6) (width 0.3) (layer F.Cu) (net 24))
 (segment (start 176.265 105.675) (end 177.8 104.14) (width 0.3) (layer F.Cu) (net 24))
 (segment (start 173.78 105.025) (end 175.645 105.025) (width 0.3) (layer F.Cu) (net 25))
 (segment (start 177.165 99.695) (end 180.34 96.52) (width 0.3) (layer F.Cu) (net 25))
 (segment (start 177.165 103.505) (end 177.165 99.695) (width 0.3) (layer F.Cu) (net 25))
 (segment (start 175.645 105.025) (end 177.165 103.505) (width 0.3) (layer F.Cu) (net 25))
 (segment (start 173.78 104.375) (end 175.025 104.375) (width 0.3) (layer F.Cu) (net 26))
 (segment (start 176.53 97.79) (end 180.34 93.98) (width 0.3) (layer F.Cu) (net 26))
 (segment (start 176.53 102.87) (end 176.53 97.79) (width 0.3) (layer F.Cu) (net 26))
 (segment (start 175.025 104.375) (end 176.53 102.87) (width 0.3) (layer F.Cu) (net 26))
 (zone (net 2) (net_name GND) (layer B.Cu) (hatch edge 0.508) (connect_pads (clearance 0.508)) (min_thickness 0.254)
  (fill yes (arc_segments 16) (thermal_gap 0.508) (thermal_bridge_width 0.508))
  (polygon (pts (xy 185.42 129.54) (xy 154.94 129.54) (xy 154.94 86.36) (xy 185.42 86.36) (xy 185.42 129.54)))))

